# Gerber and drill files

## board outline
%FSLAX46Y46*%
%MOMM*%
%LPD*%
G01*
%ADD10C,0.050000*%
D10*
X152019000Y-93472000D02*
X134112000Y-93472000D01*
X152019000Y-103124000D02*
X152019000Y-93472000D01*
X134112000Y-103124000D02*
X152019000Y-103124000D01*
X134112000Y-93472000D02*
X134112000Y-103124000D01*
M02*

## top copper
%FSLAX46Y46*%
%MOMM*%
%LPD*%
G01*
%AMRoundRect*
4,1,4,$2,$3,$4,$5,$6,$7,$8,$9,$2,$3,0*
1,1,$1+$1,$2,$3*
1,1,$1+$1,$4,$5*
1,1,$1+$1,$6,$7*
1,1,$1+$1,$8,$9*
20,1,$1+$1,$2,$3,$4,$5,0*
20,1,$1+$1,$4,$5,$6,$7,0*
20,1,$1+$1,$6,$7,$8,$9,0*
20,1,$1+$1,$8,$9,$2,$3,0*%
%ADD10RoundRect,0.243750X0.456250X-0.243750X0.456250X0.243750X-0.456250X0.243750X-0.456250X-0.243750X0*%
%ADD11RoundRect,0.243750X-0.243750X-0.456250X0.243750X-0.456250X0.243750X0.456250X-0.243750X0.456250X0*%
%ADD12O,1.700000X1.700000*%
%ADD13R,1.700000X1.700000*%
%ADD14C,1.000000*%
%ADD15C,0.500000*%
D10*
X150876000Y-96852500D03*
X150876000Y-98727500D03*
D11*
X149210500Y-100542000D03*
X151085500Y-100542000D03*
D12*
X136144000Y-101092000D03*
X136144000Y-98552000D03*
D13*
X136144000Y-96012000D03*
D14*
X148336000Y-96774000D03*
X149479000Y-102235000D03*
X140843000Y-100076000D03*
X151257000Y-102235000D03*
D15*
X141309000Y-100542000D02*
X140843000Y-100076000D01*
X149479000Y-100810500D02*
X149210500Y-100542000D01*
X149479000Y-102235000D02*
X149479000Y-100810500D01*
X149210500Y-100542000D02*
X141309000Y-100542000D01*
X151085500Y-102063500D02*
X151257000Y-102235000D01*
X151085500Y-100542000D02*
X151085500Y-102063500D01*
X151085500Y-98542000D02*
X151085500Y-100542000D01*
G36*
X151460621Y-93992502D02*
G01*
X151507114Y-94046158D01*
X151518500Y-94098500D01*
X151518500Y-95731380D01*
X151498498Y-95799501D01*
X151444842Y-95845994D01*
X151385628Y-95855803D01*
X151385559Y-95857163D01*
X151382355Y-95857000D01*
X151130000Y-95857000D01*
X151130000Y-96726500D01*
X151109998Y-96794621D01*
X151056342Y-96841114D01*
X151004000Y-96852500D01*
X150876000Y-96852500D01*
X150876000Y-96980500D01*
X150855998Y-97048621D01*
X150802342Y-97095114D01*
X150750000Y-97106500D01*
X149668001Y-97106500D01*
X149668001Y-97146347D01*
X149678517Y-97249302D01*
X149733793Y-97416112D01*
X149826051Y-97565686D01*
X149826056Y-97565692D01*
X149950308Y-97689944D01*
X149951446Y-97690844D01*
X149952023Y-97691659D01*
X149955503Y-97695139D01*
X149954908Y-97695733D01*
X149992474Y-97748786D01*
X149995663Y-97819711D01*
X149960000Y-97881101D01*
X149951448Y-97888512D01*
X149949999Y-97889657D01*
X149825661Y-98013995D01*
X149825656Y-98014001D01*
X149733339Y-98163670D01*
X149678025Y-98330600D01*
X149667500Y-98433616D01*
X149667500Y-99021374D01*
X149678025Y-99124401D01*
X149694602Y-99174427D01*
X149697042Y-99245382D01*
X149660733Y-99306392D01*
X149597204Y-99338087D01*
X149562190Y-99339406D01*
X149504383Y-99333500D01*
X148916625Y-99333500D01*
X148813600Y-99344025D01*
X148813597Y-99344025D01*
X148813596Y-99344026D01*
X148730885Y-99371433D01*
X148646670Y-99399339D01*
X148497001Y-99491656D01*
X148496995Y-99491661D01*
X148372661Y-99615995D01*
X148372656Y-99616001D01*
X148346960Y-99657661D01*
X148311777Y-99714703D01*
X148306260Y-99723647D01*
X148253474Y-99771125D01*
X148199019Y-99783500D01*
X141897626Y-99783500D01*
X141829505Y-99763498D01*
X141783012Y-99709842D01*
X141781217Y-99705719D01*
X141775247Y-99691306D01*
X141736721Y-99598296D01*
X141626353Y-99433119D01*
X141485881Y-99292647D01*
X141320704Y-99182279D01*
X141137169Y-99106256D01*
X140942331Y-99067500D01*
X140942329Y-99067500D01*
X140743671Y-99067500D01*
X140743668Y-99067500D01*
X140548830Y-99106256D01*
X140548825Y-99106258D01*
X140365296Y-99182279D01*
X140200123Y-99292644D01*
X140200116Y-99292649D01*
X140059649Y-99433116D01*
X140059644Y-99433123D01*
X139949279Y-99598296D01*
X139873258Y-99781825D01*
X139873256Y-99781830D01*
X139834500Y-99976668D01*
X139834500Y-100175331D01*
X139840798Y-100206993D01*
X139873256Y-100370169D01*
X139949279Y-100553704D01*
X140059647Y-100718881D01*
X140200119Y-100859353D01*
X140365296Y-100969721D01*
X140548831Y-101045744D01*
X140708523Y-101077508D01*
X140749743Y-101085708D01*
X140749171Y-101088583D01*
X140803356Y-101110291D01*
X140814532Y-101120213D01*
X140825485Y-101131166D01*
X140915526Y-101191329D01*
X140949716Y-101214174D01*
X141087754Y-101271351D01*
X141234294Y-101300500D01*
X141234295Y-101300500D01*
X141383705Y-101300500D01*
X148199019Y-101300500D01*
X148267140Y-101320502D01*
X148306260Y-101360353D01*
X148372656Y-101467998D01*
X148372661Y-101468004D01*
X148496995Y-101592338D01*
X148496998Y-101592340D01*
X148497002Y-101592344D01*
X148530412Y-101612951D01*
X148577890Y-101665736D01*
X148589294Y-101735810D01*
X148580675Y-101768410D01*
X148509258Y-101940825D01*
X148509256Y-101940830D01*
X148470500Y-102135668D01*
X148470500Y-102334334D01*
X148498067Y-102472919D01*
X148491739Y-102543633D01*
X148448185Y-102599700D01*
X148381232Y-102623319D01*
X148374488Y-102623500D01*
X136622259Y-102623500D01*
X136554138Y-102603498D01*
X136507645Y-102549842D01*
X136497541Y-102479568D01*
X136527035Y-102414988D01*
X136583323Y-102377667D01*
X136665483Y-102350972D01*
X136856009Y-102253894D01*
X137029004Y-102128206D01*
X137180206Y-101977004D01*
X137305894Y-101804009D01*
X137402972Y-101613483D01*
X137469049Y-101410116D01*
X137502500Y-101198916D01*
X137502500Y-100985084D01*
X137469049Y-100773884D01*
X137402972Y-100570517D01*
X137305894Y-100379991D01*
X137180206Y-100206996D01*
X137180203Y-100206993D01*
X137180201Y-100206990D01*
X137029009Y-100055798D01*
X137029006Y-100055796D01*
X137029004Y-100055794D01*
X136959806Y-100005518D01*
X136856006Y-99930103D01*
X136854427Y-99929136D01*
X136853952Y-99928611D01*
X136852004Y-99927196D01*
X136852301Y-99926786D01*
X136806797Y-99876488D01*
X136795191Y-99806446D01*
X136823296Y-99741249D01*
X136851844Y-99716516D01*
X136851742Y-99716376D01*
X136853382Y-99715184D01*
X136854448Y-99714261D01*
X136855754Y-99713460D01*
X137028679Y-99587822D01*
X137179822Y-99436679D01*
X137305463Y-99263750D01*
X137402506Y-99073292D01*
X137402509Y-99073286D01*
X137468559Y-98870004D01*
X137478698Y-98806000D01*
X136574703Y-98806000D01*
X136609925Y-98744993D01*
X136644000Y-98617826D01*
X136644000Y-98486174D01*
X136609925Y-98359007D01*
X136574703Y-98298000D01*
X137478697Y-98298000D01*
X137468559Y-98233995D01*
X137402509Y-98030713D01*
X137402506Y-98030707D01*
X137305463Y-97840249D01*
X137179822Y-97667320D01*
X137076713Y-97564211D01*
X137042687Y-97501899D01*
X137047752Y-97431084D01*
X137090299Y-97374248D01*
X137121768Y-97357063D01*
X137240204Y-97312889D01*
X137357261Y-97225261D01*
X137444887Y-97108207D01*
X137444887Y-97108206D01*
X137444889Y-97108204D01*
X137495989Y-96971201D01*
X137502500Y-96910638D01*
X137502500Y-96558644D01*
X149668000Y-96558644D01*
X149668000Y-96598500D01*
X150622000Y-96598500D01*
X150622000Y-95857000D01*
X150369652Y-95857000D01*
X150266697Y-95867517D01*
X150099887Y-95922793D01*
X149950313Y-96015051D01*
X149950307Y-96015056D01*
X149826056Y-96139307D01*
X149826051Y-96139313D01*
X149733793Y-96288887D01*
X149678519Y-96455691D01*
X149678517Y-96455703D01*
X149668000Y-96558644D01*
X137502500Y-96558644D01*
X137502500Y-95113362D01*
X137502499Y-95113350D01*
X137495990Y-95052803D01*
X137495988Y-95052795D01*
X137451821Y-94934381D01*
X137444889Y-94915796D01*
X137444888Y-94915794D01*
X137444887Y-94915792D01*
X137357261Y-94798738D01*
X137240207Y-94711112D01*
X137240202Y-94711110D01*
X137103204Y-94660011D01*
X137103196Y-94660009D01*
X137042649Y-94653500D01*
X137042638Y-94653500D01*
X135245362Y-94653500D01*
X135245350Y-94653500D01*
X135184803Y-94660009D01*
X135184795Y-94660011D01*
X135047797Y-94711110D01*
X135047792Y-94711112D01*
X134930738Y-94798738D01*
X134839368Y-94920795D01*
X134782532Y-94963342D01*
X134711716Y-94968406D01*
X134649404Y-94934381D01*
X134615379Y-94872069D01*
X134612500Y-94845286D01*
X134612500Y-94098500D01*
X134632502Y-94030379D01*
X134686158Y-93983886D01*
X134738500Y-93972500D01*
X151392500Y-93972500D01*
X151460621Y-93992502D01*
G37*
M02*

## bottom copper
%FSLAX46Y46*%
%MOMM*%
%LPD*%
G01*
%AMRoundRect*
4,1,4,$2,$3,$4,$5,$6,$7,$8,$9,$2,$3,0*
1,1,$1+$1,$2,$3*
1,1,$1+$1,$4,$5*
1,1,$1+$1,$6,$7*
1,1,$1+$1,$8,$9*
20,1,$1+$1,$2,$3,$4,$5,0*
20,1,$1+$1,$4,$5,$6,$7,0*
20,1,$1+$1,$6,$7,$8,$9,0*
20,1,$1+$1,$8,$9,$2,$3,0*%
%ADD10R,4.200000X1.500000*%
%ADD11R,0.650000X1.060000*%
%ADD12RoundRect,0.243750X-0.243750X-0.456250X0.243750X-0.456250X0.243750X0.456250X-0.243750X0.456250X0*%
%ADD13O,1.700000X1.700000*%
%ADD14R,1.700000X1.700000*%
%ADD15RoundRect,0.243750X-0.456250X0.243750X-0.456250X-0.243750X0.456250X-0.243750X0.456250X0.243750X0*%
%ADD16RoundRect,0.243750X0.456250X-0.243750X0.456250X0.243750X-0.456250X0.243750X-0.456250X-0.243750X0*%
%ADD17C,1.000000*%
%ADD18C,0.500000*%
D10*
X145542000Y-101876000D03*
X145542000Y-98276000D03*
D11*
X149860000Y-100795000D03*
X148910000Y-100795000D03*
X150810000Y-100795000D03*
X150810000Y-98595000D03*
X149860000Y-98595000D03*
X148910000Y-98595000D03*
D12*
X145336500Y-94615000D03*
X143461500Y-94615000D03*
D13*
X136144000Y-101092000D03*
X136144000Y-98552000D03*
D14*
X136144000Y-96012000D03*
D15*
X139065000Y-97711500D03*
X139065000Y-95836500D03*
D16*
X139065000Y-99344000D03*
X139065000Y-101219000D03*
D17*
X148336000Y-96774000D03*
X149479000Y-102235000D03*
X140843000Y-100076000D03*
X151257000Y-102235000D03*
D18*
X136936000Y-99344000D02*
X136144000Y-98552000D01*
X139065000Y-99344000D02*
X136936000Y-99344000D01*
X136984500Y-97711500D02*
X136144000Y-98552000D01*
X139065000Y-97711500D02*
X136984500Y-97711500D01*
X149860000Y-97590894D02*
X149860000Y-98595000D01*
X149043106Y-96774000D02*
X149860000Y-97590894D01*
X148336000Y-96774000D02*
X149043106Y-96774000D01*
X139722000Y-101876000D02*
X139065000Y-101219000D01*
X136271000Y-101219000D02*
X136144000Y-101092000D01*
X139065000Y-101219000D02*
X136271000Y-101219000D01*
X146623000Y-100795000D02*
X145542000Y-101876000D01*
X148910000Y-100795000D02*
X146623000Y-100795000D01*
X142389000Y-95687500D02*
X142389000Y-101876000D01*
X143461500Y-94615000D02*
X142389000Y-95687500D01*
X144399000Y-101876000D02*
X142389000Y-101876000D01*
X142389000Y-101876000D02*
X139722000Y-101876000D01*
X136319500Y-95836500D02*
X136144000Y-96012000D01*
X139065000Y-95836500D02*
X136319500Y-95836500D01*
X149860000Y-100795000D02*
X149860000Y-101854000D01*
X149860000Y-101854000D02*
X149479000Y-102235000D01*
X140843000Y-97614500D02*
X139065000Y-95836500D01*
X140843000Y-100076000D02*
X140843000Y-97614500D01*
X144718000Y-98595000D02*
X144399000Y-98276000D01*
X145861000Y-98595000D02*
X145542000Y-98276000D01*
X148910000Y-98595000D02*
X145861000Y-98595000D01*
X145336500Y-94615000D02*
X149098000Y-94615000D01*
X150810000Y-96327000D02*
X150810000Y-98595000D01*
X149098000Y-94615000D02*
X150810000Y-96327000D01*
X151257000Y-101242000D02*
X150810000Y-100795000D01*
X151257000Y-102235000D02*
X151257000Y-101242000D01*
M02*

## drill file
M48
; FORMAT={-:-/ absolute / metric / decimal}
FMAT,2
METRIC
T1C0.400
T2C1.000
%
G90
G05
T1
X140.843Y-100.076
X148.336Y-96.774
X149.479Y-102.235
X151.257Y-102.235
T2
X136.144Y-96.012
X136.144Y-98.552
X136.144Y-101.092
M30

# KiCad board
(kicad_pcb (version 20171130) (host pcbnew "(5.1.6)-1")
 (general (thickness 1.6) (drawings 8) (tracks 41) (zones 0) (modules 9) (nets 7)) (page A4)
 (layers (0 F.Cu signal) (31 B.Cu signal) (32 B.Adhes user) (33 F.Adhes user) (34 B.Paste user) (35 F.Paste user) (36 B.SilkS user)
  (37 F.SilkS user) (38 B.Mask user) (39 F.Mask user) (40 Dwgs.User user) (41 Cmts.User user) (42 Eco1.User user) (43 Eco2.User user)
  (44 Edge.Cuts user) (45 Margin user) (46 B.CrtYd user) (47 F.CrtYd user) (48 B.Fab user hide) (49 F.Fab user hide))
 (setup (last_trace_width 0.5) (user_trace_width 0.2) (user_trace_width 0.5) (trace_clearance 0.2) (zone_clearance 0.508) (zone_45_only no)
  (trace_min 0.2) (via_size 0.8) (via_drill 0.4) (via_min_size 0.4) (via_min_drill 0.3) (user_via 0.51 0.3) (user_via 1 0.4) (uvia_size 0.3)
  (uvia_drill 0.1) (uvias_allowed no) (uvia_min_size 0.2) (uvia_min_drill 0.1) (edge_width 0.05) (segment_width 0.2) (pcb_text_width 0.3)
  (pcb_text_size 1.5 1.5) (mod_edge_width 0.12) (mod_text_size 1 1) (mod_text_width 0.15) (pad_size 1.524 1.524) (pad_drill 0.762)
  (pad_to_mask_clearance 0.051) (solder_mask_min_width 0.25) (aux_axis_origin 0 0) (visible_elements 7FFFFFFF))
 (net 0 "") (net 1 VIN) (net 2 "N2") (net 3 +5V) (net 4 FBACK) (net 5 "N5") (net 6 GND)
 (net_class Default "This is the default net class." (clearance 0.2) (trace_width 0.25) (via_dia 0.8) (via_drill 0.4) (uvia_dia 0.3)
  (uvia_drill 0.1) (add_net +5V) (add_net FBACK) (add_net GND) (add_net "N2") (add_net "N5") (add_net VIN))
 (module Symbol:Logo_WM (layer F.Cu) (at 146.304 95.123)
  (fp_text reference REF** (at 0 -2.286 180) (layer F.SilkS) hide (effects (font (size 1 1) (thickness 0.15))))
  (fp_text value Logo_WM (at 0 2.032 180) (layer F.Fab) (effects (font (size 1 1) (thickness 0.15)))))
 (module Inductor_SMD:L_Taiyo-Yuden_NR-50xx (layer B.Cu) (at 145.542 100.076 90)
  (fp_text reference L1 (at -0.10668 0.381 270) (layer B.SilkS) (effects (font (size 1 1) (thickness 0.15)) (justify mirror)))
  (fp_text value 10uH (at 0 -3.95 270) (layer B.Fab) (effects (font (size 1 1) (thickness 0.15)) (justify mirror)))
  (pad 1 smd rect (at -1.8 0 90) (size 1.5 4.2) (layers B.Cu B.Paste B.Mask) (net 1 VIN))
  (pad 2 smd rect (at 1.8 0 90) (size 1.5 4.2) (layers B.Cu B.Paste B.Mask) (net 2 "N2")))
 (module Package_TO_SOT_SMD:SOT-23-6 (layer B.Cu) (at 149.86 99.695 270)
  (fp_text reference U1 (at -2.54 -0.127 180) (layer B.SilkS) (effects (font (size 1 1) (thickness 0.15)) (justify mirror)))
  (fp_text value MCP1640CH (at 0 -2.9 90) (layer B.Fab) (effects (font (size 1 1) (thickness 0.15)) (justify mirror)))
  (pad 5 smd rect (at 1.1 0 270) (size 1.06 0.65) (layers B.Cu B.Paste B.Mask) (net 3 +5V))
  (pad 6 smd rect (at 1.1 0.95 270) (size 1.06 0.65) (layers B.Cu B.Paste B.Mask) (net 1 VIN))
  (pad 4 smd rect (at 1.1 -0.95 270) (size 1.06 0.65) (layers B.Cu B.Paste B.Mask) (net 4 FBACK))
  (pad 3 smd rect (at -1.1 -0.95 270) (size 1.06 0.65) (layers B.Cu B.Paste B.Mask) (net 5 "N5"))
  (pad 2 smd rect (at -1.1 0 270) (size 1.06 0.65) (layers B.Cu B.Paste B.Mask) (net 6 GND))
  (pad 1 smd rect (at -1.1 0.95 270) (size 1.06 0.65) (layers B.Cu B.Paste B.Mask) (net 2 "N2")))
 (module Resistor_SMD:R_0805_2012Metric (layer F.Cu) (at 150.876 97.79 90)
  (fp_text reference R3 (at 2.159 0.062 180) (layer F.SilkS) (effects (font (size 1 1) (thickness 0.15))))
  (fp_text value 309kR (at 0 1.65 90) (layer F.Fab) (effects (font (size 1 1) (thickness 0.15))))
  (pad 2 smd roundrect (at 0.9375 0 90) (size 0.975 1.4) (layers F.Cu F.Paste F.Mask) (roundrect_rratio 0.25) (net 6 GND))
  (pad 1 smd roundrect (at -0.9375 0 90) (size 0.975 1.4) (layers F.Cu F.Paste F.Mask) (roundrect_rratio 0.25) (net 4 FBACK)))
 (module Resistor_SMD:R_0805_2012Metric (layer F.Cu) (at 150.148 100.542)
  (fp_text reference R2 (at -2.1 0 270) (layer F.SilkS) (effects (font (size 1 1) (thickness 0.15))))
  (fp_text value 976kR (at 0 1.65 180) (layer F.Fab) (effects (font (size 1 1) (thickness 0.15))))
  (pad 1 smd roundrect (at -0.9375 0) (size 0.975 1.4) (layers F.Cu F.Paste F.Mask) (roundrect_rratio 0.25) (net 3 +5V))
  (pad 2 smd roundrect (at 0.9375 0) (size 0.975 1.4) (layers F.Cu F.Paste F.Mask) (roundrect_rratio 0.25) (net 4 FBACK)))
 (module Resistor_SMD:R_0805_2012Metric (layer B.Cu) (at 144.399 94.615)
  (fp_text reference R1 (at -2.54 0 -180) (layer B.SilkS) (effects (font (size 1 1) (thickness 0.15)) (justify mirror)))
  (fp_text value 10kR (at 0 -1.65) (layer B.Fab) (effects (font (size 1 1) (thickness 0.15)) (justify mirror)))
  (pad 2 smd roundrect (at 0.9375 0) (size 0.975 1.4) (layers B.Cu B.Paste B.Mask) (roundrect_rratio 0.25) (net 5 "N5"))
  (pad 1 smd roundrect (at -0.9375 0) (size 0.975 1.4) (layers B.Cu B.Paste B.Mask) (roundrect_rratio 0.25) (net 1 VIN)))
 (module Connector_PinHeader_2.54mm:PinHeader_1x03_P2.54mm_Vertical (layer B.Cu) (at 136.144 96.012 180)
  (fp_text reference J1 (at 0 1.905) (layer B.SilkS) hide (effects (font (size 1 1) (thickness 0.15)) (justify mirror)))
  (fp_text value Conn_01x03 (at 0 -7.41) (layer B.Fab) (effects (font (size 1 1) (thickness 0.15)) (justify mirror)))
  (pad 3 thru_hole oval (at 0 -5.08 180) (size 1.7 1.7) (drill 1) (layers *.Cu *.Mask) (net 1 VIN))
  (pad 2 thru_hole oval (at 0 -2.54 180) (size 1.7 1.7) (drill 1) (layers *.Cu *.Mask) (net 6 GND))
  (pad 1 thru_hole rect (at 0 0 180) (size 1.7 1.7) (drill 1) (layers *.Cu *.Mask) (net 3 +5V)))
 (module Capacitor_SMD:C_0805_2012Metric (layer B.Cu) (at 139.065 96.774 270)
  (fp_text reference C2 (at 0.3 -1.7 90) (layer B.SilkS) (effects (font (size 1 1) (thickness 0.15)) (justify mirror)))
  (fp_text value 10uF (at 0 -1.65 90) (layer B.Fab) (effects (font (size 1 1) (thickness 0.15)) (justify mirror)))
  (pad 2 smd roundrect (at 0.9375 0 270) (size 0.975 1.4) (layers B.Cu B.Paste B.Mask) (roundrect_rratio 0.25) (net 6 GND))
  (pad 1 smd roundrect (at -0.9375 0 270) (size 0.975 1.4) (layers B.Cu B.Paste B.Mask) (roundrect_rratio 0.25) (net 3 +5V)))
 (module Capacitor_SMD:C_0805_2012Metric (layer B.Cu) (at 139.065 100.2815 90)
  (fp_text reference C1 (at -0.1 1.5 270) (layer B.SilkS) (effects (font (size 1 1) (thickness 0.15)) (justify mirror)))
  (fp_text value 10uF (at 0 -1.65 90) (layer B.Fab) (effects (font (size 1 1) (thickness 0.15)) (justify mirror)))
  (pad 2 smd roundrect (at 0.9375 0 90) (size 0.975 1.4) (layers B.Cu B.Paste B.Mask) (roundrect_rratio 0.25) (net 6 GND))
  (pad 1 smd roundrect (at -0.9375 0 90) (size 0.975 1.4) (layers B.Cu B.Paste B.Mask) (roundrect_rratio 0.25) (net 1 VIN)))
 (gr_line (start 152.019 93.472) (end 134.112 93.472) (layer Edge.Cuts) (width 0.05))
 (gr_line (start 152.019 103.124) (end 152.019 93.472) (layer Edge.Cuts) (width 0.05))
 (gr_line (start 134.112 103.124) (end 152.019 103.124) (layer Edge.Cuts) (width 0.05))
 (gr_line (start 134.112 93.472) (end 134.112 103.124) (layer Edge.Cuts) (width 0.05))
 (segment (start 136.936 99.344) (end 136.144 98.552) (width 0.5) (layer B.Cu) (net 6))
 (segment (start 139.065 99.344) (end 136.936 99.344) (width 0.5) (layer B.Cu) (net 6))
 (segment (start 136.9845 97.7115) (end 136.144 98.552) (width 0.5) (layer B.Cu) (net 6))
 (segment (start 139.065 97.7115) (end 136.9845 97.7115) (width 0.5) (layer B.Cu) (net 6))
 (via (at 148.336 96.774) (size 1) (drill 0.4) (layers F.Cu B.Cu) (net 6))
 (segment (start 149.86 97.590894) (end 149.86 98.595) (width 0.5) (layer B.Cu) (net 6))
 (segment (start 149.043106 96.774) (end 149.86 97.590894) (width 0.5) (layer B.Cu) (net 6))
 (segment (start 148.336 96.774) (end 149.043106 96.774) (width 0.5) (layer B.Cu) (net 6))
 (segment (start 139.722 101.876) (end 139.065 101.219) (width 0.5) (layer B.Cu) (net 1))
 (segment (start 136.271 101.219) (end 136.144 101.092) (width 0.5) (layer B.Cu) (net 1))
 (segment (start 139.065 101.219) (end 136.271 101.219) (width 0.5) (layer B.Cu) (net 1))
 (segment (start 146.623 100.795) (end 145.542 101.876) (width 0.5) (layer B.Cu) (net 1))
 (segment (start 148.91 100.795) (end 146.623 100.795) (width 0.5) (layer B.Cu) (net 1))
 (segment (start 142.389 95.6875) (end 142.389 101.876) (width 0.5) (layer B.Cu) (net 1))
 (segment (start 143.4615 94.615) (end 142.389 95.6875) (width 0.5) (layer B.Cu) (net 1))
 (segment (start 144.399 101.876) (end 142.389 101.876) (width 0.5) (layer B.Cu) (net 1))
 (segment (start 142.389 101.876) (end 139.722 101.876) (width 0.5) (layer B.Cu) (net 1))
 (segment (start 136.3195 95.8365) (end 136.144 96.012) (width 0.5) (layer B.Cu) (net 3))
 (segment (start 139.065 95.8365) (end 136.3195 95.8365) (width 0.5) (layer B.Cu) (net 3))
 (via (at 149.479 102.235) (size 1) (drill 0.4) (layers F.Cu B.Cu) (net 3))
 (segment (start 149.86 100.795) (end 149.86 101.854) (width 0.5) (layer B.Cu) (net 3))
 (segment (start 149.86 101.854) (end 149.479 102.235) (width 0.5) (layer B.Cu) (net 3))
 (via (at 140.843 100.076) (size 1) (drill 0.4) (layers F.Cu B.Cu) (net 3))
 (segment (start 141.309 100.542) (end 140.843 100.076) (width 0.5) (layer F.Cu) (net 3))
 (segment (start 140.843 97.6145) (end 139.065 95.8365) (width 0.5) (layer B.Cu) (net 3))
 (segment (start 140.843 100.076) (end 140.843 97.6145) (width 0.5) (layer B.Cu) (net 3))
 (segment (start 149.479 100.8105) (end 149.2105 100.542) (width 0.5) (layer F.Cu) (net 3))
 (segment (start 149.479 102.235) (end 149.479 100.8105) (width 0.5) (layer F.Cu) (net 3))
 (segment (start 149.2105 100.542) (end 141.309 100.542) (width 0.5) (layer F.Cu) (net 3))
 (segment (start 144.718 98.595) (end 144.399 98.276) (width 0.5) (layer B.Cu) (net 2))
 (segment (start 145.861 98.595) (end 145.542 98.276) (width 0.5) (layer B.Cu) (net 2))
 (segment (start 148.91 98.595) (end 145.861 98.595) (width 0.5) (layer B.Cu) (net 2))
 (segment (start 145.3365 94.615) (end 149.098 94.615) (width 0.5) (layer B.Cu) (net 5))
 (segment (start 150.81 96.327) (end 150.81 98.595) (width 0.5) (layer B.Cu) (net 5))
 (segment (start 149.098 94.615) (end 150.81 96.327) (width 0.5) (layer B.Cu) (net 5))
 (via (at 151.257 102.235) (size 1) (drill 0.4) (layers F.Cu B.Cu) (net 4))
 (segment (start 151.257 101.242) (end 150.81 100.795) (width 0.5) (layer B.Cu) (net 4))
 (segment (start 151.257 102.235) (end 151.257 101.242) (width 0.5) (layer B.Cu) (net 4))
 (segment (start 151.0855 102.0635) (end 151.257 102.235) (width 0.5) (layer F.Cu) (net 4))
 (segment (start 151.0855 100.542) (end 151.0855 102.0635) (width 0.5) (layer F.Cu) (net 4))
 (segment (start 151.0855 98.542) (end 151.0855 100.542) (width 0.5) (layer F.Cu) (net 4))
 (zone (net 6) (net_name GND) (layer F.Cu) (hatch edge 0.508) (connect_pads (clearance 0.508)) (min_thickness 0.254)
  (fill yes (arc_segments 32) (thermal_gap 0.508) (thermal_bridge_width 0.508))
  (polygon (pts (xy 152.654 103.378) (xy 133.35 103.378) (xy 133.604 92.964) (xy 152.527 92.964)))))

